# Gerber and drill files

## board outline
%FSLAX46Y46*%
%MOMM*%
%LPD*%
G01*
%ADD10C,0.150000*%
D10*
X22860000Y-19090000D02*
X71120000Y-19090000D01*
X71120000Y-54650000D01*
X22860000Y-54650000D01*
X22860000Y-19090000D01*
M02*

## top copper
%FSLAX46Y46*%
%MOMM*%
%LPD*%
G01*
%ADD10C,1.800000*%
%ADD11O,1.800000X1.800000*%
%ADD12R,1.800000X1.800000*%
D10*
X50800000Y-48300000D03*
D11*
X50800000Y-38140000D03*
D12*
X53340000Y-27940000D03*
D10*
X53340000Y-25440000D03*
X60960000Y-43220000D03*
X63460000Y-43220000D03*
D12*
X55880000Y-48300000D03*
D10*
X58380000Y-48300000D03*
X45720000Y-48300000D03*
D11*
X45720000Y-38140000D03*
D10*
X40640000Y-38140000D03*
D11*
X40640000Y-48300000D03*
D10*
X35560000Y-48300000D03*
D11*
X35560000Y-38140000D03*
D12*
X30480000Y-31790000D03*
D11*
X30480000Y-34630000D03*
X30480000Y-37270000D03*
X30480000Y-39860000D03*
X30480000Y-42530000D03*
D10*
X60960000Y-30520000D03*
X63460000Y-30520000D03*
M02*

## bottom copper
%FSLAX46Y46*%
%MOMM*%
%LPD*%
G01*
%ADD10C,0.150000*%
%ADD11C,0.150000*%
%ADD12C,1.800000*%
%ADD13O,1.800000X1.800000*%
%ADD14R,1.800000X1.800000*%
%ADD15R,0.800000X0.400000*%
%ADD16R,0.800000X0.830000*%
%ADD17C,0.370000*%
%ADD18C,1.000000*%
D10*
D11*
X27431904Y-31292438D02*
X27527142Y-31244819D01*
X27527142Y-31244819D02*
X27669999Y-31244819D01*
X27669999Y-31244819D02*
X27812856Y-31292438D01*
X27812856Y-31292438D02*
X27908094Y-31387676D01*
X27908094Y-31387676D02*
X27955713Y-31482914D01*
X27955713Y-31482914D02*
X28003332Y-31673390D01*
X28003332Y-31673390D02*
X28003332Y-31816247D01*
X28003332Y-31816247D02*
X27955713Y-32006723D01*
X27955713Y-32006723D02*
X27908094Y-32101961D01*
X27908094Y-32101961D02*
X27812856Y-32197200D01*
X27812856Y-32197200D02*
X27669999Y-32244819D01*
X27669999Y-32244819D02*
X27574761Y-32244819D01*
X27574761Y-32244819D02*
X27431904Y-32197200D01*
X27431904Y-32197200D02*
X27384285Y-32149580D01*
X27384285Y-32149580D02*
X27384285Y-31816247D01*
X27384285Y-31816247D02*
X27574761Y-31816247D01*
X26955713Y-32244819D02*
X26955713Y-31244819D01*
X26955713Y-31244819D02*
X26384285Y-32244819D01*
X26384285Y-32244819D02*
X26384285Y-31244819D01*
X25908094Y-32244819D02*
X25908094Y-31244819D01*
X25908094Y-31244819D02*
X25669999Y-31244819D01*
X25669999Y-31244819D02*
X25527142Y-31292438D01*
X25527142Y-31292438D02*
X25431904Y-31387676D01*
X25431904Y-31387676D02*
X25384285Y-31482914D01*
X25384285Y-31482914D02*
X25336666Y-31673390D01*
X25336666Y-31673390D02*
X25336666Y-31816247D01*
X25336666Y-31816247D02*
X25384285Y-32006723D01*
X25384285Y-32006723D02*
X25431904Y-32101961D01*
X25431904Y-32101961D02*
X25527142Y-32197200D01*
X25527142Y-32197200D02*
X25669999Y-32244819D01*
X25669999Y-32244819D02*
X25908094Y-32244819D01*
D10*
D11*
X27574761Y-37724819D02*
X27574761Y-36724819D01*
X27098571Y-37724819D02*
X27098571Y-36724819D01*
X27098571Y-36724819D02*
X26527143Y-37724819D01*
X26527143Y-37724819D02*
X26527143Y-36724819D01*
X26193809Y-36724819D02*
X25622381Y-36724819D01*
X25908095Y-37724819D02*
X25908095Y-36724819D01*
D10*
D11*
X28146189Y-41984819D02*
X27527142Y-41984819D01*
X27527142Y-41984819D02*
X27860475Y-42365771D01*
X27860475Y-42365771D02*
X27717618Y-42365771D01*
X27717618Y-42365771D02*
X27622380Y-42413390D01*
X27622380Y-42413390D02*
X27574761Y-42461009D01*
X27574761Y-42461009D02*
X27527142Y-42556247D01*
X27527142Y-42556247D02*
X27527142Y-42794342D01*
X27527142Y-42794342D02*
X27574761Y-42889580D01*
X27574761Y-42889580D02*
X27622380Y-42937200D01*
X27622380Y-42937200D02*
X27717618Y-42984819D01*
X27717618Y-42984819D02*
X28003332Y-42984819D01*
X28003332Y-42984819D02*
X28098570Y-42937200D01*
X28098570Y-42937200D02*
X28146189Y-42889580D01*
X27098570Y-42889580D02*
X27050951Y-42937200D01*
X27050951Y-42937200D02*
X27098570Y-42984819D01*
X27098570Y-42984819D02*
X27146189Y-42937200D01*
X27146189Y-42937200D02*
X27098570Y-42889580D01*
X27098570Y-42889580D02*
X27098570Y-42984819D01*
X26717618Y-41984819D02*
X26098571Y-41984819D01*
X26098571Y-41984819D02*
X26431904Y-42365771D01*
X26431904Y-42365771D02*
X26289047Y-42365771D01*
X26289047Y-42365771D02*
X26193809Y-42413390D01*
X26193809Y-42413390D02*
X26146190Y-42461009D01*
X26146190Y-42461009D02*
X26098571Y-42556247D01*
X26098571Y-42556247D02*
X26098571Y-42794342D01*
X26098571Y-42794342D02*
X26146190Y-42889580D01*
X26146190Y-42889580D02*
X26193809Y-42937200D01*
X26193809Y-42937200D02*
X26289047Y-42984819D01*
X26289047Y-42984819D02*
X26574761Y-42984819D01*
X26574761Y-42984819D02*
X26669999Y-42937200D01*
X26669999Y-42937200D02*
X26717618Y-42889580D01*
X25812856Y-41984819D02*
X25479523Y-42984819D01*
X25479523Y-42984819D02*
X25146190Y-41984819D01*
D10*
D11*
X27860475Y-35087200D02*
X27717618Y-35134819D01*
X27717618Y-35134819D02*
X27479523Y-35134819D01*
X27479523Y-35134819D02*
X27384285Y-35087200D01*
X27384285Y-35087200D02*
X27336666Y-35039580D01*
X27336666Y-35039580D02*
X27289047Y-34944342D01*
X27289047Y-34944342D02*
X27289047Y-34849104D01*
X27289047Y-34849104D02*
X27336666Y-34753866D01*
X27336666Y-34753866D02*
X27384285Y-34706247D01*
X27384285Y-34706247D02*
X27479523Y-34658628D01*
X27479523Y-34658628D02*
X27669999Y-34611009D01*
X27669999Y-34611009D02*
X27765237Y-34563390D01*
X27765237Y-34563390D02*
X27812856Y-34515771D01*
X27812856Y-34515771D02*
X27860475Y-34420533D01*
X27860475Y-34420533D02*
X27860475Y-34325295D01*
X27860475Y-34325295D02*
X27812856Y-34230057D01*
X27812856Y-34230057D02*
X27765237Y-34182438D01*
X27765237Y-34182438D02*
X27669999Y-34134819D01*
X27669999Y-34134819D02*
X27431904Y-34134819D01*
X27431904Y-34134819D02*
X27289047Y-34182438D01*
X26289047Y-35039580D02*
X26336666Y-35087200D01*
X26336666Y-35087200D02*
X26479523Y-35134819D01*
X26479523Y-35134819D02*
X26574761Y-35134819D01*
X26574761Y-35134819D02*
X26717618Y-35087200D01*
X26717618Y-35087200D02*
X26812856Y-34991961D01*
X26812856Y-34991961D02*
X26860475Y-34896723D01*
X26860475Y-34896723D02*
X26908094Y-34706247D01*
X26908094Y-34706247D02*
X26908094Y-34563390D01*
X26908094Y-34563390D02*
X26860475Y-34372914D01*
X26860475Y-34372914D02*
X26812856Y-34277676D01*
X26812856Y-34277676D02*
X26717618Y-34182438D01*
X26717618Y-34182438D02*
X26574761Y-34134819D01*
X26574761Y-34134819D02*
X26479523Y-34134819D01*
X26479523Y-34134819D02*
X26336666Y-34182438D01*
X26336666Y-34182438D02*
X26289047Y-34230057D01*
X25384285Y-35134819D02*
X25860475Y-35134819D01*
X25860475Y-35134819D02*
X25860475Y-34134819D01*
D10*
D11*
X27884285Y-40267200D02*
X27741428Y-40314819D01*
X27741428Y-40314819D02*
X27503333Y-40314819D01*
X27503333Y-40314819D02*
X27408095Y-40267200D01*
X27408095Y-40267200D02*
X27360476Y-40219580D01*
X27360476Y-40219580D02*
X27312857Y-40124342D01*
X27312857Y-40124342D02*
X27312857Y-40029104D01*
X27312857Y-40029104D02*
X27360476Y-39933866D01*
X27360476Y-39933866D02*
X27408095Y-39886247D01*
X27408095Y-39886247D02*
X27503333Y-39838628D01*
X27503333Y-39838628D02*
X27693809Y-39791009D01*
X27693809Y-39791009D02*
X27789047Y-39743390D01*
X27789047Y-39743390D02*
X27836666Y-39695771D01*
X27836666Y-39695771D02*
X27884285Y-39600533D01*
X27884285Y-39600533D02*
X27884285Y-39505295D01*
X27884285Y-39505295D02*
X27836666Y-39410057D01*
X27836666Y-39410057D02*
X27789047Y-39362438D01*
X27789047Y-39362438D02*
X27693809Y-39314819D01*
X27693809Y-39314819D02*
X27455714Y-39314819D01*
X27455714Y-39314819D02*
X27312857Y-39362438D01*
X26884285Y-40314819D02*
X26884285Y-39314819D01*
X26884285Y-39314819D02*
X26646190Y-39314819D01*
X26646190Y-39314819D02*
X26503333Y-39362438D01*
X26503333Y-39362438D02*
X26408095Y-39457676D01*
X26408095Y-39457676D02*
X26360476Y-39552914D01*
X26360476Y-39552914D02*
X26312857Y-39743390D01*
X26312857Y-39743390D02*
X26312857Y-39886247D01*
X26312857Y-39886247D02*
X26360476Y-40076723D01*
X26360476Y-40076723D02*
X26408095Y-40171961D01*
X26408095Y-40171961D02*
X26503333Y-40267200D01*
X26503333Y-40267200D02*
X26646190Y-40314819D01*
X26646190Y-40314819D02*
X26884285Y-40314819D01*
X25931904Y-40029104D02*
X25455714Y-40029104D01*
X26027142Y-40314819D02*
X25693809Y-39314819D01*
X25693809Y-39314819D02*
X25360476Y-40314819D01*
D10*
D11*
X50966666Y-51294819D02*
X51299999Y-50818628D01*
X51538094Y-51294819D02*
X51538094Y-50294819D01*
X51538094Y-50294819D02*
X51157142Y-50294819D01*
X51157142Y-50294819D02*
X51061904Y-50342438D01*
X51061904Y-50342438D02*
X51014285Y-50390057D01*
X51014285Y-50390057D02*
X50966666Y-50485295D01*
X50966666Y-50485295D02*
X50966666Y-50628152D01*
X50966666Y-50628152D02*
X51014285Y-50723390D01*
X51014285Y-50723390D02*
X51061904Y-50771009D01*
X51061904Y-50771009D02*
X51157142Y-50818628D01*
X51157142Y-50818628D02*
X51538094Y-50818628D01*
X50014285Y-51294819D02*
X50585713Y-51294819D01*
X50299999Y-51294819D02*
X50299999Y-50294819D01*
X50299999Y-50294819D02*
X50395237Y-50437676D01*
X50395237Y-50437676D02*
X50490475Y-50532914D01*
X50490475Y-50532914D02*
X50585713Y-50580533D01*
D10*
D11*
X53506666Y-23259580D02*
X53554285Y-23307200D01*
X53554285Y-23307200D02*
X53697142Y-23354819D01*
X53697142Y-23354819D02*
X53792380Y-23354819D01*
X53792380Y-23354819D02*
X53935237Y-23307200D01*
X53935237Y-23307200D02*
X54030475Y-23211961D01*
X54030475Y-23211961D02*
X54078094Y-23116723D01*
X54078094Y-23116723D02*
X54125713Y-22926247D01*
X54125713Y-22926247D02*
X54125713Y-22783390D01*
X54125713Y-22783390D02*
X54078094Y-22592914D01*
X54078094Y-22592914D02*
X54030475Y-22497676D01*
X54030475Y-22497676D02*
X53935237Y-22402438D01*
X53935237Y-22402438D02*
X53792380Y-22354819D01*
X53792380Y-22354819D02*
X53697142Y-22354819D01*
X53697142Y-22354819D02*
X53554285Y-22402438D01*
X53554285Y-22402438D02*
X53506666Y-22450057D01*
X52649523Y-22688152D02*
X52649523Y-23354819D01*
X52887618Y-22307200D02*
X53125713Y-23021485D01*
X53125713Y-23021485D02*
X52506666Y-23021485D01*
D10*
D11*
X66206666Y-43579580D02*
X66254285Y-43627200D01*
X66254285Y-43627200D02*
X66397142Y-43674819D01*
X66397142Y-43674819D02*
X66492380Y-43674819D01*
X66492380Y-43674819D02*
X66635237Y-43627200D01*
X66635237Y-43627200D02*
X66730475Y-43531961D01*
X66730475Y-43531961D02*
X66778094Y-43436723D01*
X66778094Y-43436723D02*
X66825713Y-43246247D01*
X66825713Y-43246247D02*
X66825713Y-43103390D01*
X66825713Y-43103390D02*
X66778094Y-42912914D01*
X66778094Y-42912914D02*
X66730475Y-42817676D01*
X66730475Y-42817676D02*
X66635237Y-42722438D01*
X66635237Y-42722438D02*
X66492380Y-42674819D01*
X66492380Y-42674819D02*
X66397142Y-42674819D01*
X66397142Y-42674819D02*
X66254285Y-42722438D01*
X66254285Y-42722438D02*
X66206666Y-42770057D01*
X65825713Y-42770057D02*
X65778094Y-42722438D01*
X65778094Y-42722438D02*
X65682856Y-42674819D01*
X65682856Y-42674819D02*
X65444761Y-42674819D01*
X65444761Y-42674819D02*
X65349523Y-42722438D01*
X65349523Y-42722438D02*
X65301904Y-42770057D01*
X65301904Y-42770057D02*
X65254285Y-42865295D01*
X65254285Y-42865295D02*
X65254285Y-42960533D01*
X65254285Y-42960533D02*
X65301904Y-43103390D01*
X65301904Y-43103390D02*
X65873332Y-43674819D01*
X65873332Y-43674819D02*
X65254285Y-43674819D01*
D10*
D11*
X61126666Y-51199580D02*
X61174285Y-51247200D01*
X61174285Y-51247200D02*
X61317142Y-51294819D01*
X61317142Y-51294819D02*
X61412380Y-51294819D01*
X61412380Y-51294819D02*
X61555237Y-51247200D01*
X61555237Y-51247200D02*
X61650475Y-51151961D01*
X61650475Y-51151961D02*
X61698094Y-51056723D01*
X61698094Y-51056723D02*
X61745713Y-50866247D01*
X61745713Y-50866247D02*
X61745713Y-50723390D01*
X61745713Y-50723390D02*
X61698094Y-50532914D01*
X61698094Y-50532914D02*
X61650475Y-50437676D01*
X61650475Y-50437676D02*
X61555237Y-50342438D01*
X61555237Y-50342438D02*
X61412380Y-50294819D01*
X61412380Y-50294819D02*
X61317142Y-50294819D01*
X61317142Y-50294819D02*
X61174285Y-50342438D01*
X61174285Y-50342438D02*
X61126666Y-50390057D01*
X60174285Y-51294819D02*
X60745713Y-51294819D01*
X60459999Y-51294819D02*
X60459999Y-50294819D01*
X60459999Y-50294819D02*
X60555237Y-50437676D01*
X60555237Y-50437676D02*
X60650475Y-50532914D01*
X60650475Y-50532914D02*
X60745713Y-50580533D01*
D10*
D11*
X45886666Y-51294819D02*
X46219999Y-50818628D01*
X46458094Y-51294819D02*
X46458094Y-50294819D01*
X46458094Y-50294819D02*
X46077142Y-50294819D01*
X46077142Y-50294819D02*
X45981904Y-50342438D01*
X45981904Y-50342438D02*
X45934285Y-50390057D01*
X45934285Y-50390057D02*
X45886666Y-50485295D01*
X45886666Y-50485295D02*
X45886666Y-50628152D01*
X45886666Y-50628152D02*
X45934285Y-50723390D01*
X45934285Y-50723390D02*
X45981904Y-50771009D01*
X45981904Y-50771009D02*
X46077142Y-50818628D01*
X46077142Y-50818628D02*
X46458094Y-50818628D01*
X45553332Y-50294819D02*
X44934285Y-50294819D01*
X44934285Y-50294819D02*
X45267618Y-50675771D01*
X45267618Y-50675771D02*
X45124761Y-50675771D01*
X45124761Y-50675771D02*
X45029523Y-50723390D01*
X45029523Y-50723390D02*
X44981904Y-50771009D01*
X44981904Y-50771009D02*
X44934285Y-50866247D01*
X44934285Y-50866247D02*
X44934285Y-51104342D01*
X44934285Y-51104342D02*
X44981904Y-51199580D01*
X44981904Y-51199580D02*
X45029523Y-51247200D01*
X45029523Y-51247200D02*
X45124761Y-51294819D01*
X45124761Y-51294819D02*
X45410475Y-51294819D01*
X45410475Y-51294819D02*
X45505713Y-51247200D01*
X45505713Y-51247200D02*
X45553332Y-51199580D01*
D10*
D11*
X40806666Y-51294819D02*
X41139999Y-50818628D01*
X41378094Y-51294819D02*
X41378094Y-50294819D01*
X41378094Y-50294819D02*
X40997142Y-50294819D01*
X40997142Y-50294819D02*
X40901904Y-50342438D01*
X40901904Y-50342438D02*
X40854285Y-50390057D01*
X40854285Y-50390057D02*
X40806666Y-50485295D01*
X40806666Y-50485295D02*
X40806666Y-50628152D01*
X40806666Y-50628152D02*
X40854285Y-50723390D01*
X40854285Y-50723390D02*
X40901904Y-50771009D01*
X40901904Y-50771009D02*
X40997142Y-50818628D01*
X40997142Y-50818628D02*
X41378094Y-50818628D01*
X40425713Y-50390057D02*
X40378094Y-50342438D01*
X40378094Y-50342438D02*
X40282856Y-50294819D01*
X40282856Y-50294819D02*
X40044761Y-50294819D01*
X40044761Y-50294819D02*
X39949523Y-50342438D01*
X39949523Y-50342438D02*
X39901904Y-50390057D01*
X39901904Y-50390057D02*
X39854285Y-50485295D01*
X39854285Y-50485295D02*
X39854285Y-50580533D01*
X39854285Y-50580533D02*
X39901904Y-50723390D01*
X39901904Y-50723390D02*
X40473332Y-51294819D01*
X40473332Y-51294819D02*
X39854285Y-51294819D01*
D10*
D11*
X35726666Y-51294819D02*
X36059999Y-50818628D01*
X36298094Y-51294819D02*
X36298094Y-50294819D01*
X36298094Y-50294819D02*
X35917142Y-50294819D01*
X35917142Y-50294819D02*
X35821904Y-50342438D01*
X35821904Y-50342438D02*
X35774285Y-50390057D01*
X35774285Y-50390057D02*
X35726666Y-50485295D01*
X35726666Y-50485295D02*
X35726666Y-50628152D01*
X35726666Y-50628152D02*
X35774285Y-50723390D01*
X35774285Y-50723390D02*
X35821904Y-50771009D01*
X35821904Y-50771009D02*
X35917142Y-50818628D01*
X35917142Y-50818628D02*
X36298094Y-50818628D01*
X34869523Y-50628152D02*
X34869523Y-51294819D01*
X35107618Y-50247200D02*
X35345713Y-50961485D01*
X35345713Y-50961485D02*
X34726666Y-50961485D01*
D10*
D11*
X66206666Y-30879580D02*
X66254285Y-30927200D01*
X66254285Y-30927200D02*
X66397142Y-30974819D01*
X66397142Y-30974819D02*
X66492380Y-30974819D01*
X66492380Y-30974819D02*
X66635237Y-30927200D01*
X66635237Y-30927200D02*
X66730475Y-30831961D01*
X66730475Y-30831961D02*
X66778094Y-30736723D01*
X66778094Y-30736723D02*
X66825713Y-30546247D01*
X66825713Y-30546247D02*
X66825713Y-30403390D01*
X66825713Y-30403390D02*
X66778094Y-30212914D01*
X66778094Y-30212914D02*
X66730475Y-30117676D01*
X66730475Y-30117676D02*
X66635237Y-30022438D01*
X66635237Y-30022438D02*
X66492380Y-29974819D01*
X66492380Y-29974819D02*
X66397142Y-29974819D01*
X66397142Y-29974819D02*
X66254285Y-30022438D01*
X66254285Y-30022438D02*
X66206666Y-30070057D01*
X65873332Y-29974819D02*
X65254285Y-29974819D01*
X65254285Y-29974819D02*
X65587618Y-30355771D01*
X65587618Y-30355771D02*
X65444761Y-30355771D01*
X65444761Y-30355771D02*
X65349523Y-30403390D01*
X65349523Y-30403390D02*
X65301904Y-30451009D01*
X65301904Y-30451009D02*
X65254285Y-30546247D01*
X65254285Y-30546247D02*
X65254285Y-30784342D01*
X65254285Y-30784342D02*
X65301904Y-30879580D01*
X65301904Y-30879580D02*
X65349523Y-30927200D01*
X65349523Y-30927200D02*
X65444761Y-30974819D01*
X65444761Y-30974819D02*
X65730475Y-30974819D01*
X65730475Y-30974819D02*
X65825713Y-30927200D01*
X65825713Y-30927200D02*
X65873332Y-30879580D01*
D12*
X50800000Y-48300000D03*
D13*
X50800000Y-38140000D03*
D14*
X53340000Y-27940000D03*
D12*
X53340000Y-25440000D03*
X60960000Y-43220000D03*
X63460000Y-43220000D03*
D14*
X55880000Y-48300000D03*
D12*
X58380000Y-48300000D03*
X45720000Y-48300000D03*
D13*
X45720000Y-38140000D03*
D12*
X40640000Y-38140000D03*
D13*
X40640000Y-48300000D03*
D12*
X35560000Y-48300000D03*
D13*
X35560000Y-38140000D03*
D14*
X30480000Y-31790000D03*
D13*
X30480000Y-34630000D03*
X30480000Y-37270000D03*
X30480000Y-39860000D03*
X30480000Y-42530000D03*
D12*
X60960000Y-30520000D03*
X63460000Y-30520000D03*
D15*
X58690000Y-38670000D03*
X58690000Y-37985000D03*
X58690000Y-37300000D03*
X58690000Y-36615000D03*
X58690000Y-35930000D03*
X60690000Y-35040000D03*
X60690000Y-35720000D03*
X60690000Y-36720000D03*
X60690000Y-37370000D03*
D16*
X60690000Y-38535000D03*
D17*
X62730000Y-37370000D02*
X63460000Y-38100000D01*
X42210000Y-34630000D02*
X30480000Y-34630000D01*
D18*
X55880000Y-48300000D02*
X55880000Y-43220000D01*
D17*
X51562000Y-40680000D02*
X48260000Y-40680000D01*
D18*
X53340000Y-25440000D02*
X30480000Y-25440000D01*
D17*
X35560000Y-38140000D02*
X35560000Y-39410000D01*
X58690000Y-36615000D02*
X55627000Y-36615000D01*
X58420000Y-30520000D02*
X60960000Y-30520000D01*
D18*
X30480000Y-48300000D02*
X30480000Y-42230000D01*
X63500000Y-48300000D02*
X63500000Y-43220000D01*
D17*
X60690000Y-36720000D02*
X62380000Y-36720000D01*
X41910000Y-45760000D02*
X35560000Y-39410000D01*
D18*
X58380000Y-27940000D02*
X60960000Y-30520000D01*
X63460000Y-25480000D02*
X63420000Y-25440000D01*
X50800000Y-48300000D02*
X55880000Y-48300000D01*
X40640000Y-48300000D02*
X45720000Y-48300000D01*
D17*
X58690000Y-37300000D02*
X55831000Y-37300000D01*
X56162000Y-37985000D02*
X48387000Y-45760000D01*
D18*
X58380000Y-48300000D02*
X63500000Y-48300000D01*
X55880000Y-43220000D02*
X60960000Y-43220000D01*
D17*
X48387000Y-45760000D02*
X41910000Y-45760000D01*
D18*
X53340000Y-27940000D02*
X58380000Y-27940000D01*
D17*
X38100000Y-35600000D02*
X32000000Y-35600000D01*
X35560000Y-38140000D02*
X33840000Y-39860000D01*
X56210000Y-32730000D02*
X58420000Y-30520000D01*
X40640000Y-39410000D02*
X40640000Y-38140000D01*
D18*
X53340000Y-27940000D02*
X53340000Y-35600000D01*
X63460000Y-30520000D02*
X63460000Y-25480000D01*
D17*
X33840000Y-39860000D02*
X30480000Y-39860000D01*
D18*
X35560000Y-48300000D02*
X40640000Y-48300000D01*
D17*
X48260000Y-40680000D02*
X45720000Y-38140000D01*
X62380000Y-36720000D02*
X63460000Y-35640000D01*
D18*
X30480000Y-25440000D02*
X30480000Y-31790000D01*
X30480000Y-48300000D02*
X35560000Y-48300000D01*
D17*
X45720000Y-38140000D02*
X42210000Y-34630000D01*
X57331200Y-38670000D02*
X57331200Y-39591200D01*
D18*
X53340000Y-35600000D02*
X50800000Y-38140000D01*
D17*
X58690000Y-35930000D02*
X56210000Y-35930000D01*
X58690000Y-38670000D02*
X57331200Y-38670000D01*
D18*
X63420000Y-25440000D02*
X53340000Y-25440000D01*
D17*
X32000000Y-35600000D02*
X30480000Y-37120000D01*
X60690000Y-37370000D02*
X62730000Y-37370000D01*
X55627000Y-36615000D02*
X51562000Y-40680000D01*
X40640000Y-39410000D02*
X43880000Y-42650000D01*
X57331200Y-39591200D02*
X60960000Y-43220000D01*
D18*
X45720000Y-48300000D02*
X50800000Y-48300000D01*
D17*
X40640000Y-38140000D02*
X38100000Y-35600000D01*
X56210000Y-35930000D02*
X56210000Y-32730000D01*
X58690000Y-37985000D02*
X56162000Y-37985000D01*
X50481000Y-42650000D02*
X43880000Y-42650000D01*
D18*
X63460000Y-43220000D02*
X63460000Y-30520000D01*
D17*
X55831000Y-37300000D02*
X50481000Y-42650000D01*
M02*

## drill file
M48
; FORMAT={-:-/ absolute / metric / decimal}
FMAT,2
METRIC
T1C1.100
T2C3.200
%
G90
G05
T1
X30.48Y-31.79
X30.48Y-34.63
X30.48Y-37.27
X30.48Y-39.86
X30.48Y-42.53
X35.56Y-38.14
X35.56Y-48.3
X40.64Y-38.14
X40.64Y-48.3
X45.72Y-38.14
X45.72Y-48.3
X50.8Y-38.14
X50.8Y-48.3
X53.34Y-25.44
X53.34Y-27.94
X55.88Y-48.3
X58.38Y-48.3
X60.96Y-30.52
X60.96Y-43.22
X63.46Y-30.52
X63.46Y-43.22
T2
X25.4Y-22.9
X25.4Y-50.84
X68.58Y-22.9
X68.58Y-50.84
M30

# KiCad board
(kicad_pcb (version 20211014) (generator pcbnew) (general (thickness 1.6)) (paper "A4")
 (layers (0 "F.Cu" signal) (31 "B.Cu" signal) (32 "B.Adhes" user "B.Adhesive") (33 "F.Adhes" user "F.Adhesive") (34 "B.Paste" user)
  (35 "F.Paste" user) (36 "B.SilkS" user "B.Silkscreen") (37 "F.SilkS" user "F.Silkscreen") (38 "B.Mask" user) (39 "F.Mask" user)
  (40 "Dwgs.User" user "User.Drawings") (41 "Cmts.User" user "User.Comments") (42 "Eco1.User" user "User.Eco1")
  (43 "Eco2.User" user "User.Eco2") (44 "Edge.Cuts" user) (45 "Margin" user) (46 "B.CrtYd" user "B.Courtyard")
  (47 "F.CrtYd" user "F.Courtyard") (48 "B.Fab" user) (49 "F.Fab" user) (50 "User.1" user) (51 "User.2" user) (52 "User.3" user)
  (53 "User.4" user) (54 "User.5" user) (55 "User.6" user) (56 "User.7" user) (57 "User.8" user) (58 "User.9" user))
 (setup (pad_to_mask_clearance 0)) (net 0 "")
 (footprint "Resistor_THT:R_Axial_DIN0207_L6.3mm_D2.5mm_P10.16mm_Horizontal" (layer "F.Cu") (at 50.8 48.3 90)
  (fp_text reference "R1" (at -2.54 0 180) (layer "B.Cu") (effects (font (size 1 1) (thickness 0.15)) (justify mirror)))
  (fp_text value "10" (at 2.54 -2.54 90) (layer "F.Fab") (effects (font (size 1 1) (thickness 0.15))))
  (pad "1" thru_hole circle (at 0 0 90) (size 1.8 1.8) (drill 1.1) (layers *.Cu *.Mask))
  (pad "2" thru_hole oval (at 10.16 0 90) (size 1.8 1.8) (drill 1.1) (layers *.Cu *.Mask)))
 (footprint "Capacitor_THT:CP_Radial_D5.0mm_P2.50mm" (layer "F.Cu") (at 53.34 27.94 90)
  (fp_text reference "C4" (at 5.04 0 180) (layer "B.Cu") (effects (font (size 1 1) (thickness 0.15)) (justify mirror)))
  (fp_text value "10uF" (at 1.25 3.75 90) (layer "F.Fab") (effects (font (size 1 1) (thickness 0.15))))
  (pad "1" thru_hole rect (at 0 0 90) (size 1.8 1.8) (drill 1.1) (layers *.Cu *.Mask))
  (pad "2" thru_hole circle (at 2.5 0 90) (size 1.8 1.8) (drill 1.1) (layers *.Cu *.Mask)))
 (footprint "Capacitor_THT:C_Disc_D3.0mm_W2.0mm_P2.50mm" (layer "F.Cu") (at 60.96 43.22)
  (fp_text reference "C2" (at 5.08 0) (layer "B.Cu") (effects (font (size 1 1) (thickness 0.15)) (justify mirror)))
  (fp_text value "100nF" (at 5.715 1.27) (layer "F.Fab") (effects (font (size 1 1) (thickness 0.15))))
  (pad "1" thru_hole circle (at 0 0) (size 1.8 1.8) (drill 1.1) (layers *.Cu *.Mask))
  (pad "2" thru_hole circle (at 2.5 0) (size 1.8 1.8) (drill 1.1) (layers *.Cu *.Mask)))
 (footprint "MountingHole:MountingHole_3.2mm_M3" (layer "F.Cu") (at 25.4 22.9)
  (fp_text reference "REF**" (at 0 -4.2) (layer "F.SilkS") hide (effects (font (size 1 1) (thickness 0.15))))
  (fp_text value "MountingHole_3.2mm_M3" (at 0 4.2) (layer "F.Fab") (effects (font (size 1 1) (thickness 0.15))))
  (pad "" np_thru_hole circle (at 0 0) (size 3.2 3.2) (drill 3.2) (layers *.Cu *.Mask)))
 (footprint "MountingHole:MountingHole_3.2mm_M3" (layer "F.Cu") (at 25.4 50.84)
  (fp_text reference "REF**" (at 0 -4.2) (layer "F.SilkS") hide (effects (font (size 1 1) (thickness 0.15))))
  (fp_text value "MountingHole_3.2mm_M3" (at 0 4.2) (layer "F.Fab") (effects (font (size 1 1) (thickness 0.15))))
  (pad "" np_thru_hole circle (at 0 0) (size 3.2 3.2) (drill 3.2) (layers *.Cu *.Mask)))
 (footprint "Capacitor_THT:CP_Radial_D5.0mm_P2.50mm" (layer "F.Cu") (at 55.88 48.3)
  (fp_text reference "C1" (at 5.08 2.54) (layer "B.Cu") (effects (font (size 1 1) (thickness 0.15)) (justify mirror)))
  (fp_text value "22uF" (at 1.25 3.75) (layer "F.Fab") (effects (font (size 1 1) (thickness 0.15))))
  (pad "1" thru_hole rect (at 0 0) (size 1.8 1.8) (drill 1.1) (layers *.Cu *.Mask))
  (pad "2" thru_hole circle (at 2.5 0) (size 1.8 1.8) (drill 1.1) (layers *.Cu *.Mask)))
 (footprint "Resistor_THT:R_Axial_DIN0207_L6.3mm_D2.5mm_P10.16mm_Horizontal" (layer "F.Cu") (at 45.72 48.3 90)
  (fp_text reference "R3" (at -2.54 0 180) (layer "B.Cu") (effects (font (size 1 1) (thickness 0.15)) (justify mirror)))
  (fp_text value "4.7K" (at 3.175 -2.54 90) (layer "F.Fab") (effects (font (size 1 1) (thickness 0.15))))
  (pad "1" thru_hole circle (at 0 0 90) (size 1.8 1.8) (drill 1.1) (layers *.Cu *.Mask))
  (pad "2" thru_hole oval (at 10.16 0 90) (size 1.8 1.8) (drill 1.1) (layers *.Cu *.Mask)))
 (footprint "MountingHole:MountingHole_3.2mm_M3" (layer "F.Cu") (at 68.58 22.9)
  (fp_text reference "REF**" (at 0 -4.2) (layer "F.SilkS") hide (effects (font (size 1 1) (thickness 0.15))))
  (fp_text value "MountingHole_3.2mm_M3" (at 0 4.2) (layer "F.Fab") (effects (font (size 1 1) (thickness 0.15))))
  (pad "" np_thru_hole circle (at 0 0) (size 3.2 3.2) (drill 3.2) (layers *.Cu *.Mask)))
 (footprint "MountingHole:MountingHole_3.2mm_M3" (layer "F.Cu") (at 68.58 50.84)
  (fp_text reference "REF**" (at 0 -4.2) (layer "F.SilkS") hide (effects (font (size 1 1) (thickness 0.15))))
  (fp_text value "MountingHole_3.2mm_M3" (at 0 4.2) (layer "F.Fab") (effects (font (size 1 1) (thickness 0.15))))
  (pad "" np_thru_hole circle (at 0 0) (size 3.2 3.2) (drill 3.2) (layers *.Cu *.Mask)))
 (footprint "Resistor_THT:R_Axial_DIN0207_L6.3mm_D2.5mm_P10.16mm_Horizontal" (layer "F.Cu") (at 40.64 38.14 -90)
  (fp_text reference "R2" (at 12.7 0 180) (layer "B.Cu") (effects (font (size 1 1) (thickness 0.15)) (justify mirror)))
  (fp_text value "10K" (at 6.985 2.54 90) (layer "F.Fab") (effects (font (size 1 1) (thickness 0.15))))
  (pad "1" thru_hole circle (at 0 0 270) (size 1.8 1.8) (drill 1.1) (layers *.Cu *.Mask))
  (pad "2" thru_hole oval (at 10.16 0 270) (size 1.8 1.8) (drill 1.1) (layers *.Cu *.Mask)))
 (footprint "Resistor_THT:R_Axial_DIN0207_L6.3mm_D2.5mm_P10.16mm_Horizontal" (layer "F.Cu") (at 35.56 48.3 90)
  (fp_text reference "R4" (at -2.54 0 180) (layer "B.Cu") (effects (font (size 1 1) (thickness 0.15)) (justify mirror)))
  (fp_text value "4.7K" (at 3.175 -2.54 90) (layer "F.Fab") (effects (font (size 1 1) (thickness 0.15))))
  (pad "1" thru_hole circle (at 0 0 90) (size 1.8 1.8) (drill 1.1) (layers *.Cu *.Mask))
  (pad "2" thru_hole oval (at 10.16 0 90) (size 1.8 1.8) (drill 1.1) (layers *.Cu *.Mask)))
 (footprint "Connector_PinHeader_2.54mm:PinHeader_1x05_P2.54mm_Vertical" (layer "F.Cu") (at 30.48 31.79)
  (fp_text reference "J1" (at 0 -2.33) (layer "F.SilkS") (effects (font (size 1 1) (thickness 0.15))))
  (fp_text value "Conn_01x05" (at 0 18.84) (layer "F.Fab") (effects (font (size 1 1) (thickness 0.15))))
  (pad "1" thru_hole rect (at 0 0) (size 1.8 1.8) (drill 1.1) (layers *.Cu *.Mask))
  (pad "2" thru_hole oval (at 0 2.84) (size 1.8 1.8) (drill 1.1) (layers *.Cu *.Mask))
  (pad "3" thru_hole oval (at 0 5.48) (size 1.8 1.8) (drill 1.1) (layers *.Cu *.Mask))
  (pad "4" thru_hole oval (at 0 8.07) (size 1.8 1.8) (drill 1.1) (layers *.Cu *.Mask))
  (pad "5" thru_hole oval (at 0 10.74) (size 1.8 1.8) (drill 1.1) (layers *.Cu *.Mask)))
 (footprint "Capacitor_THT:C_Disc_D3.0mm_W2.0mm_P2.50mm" (layer "F.Cu") (at 60.96 30.52)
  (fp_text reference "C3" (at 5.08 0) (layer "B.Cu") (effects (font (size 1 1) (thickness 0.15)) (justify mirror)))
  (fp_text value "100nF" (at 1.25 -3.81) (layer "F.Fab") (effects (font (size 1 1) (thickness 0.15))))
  (pad "1" thru_hole circle (at 0 0) (size 1.8 1.8) (drill 1.1) (layers *.Cu *.Mask))
  (pad "2" thru_hole circle (at 2.5 0) (size 1.8 1.8) (drill 1.1) (layers *.Cu *.Mask)))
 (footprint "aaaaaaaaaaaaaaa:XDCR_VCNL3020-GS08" (layer "B.Cu") (at 59.69 36.87)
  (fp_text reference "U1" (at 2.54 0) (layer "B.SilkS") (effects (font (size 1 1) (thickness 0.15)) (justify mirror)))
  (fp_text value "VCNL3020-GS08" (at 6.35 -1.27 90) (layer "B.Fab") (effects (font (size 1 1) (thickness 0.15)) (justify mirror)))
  (pad "1" smd rect (at -1 1.8 270) (size 0.4 0.8) (layers "B.Cu" "B.Paste" "B.Mask"))
  (pad "2" smd rect (at -1 1.115 90) (size 0.4 0.8) (layers "B.Cu" "B.Paste" "B.Mask"))
  (pad "3" smd rect (at -1 0.43 90) (size 0.4 0.8) (layers "B.Cu" "B.Paste" "B.Mask"))
  (pad "4" smd rect (at -1 -0.255 90) (size 0.4 0.8) (layers "B.Cu" "B.Paste" "B.Mask"))
  (pad "5" smd rect (at -1 -0.94 90) (size 0.4 0.8) (layers "B.Cu" "B.Paste" "B.Mask"))
  (pad "6" smd rect (at 1 -1.83 270) (size 0.4 0.8) (layers "B.Cu" "B.Paste" "B.Mask"))
  (pad "7" smd rect (at 1 -1.15 270) (size 0.4 0.8) (layers "B.Cu" "B.Paste" "B.Mask"))
  (pad "8" smd rect (at 1 -0.15 270) (size 0.4 0.8) (layers "B.Cu" "B.Paste" "B.Mask"))
  (pad "9" smd rect (at 1 0.5 270) (size 0.4 0.8) (layers "B.Cu" "B.Paste" "B.Mask"))
  (pad "10" smd rect (at 1 1.665 270) (size 0.83 0.8) (layers "B.Cu" "B.Paste" "B.Mask")))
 (gr_rect (start 22.86 19.09) (end 71.12 54.65) (layer "Edge.Cuts") (width 0.15) (fill none))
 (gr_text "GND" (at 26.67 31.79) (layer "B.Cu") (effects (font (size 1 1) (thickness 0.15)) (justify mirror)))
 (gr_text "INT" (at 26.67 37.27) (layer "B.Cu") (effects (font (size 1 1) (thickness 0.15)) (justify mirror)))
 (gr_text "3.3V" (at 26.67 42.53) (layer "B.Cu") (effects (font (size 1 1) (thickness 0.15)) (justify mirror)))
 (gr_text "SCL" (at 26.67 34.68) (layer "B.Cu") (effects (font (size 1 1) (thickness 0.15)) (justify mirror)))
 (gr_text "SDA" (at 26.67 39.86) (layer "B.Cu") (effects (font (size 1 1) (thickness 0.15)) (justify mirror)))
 (segment (start 62.73 37.37) (end 63.46 38.1) (width 0.37) (layer "B.Cu") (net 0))
 (segment (start 42.21 34.63) (end 30.48 34.63) (width 0.37) (layer "B.Cu") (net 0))
 (segment (start 55.88 48.3) (end 55.88 43.22) (width 1) (layer "B.Cu") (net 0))
 (segment (start 51.562 40.68) (end 48.26 40.68) (width 0.37) (layer "B.Cu") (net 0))
 (segment (start 53.34 25.44) (end 30.48 25.44) (width 1) (layer "B.Cu") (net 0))
 (segment (start 35.56 38.14) (end 35.56 39.41) (width 0.37) (layer "B.Cu") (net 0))
 (segment (start 58.69 36.615) (end 55.627 36.615) (width 0.37) (layer "B.Cu") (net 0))
 (segment (start 58.42 30.52) (end 60.96 30.52) (width 0.37) (layer "B.Cu") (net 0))
 (segment (start 30.48 48.3) (end 30.48 42.23) (width 1) (layer "B.Cu") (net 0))
 (segment (start 63.5 48.3) (end 63.5 43.22) (width 1) (layer "B.Cu") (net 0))
 (segment (start 60.69 36.72) (end 62.38 36.72) (width 0.37) (layer "B.Cu") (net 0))
 (segment (start 41.91 45.76) (end 35.56 39.41) (width 0.37) (layer "B.Cu") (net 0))
 (segment (start 58.38 27.94) (end 60.96 30.52) (width 1) (layer "B.Cu") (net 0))
 (segment (start 63.46 25.48) (end 63.42 25.44) (width 1) (layer "B.Cu") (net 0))
 (segment (start 50.8 48.3) (end 55.88 48.3) (width 1) (layer "B.Cu") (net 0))
 (segment (start 40.64 48.3) (end 45.72 48.3) (width 1) (layer "B.Cu") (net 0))
 (segment (start 58.69 37.3) (end 55.831 37.3) (width 0.37) (layer "B.Cu") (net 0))
 (segment (start 56.162 37.985) (end 48.387 45.76) (width 0.37) (layer "B.Cu") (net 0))
 (segment (start 58.38 48.3) (end 63.5 48.3) (width 1) (layer "B.Cu") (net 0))
 (segment (start 55.88 43.22) (end 60.96 43.22) (width 1) (layer "B.Cu") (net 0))
 (segment (start 48.387 45.76) (end 41.91 45.76) (width 0.37) (layer "B.Cu") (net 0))
 (segment (start 53.34 27.94) (end 58.38 27.94) (width 1) (layer "B.Cu") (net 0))
 (segment (start 38.1 35.6) (end 32 35.6) (width 0.37) (layer "B.Cu") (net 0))
 (segment (start 35.56 38.14) (end 33.84 39.86) (width 0.37) (layer "B.Cu") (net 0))
 (segment (start 56.21 32.73) (end 58.42 30.52) (width 0.37) (layer "B.Cu") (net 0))
 (segment (start 40.64 39.41) (end 40.64 38.14) (width 0.37) (layer "B.Cu") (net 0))
 (segment (start 53.34 27.94) (end 53.34 35.6) (width 1) (layer "B.Cu") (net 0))
 (segment (start 63.46 30.52) (end 63.46 25.48) (width 1) (layer "B.Cu") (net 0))
 (segment (start 33.84 39.86) (end 30.48 39.86) (width 0.37) (layer "B.Cu") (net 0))
 (segment (start 35.56 48.3) (end 40.64 48.3) (width 1) (layer "B.Cu") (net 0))
 (segment (start 48.26 40.68) (end 45.72 38.14) (width 0.37) (layer "B.Cu") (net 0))
 (segment (start 62.38 36.72) (end 63.46 35.64) (width 0.37) (layer "B.Cu") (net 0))
 (segment (start 30.48 25.44) (end 30.48 31.79) (width 1) (layer "B.Cu") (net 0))
 (segment (start 30.48 48.3) (end 35.56 48.3) (width 1) (layer "B.Cu") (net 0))
 (segment (start 45.72 38.14) (end 42.21 34.63) (width 0.37) (layer "B.Cu") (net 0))
 (segment (start 57.3312 38.67) (end 57.3312 39.5912) (width 0.37) (layer "B.Cu") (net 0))
 (segment (start 53.34 35.6) (end 50.8 38.14) (width 1) (layer "B.Cu") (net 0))
 (segment (start 58.69 35.93) (end 56.21 35.93) (width 0.37) (layer "B.Cu") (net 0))
 (segment (start 58.69 38.67) (end 57.3312 38.67) (width 0.37) (layer "B.Cu") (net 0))
 (segment (start 63.42 25.44) (end 53.34 25.44) (width 1) (layer "B.Cu") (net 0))
 (segment (start 32 35.6) (end 30.48 37.12) (width 0.37) (layer "B.Cu") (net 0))
 (segment (start 60.69 37.37) (end 62.73 37.37) (width 0.37) (layer "B.Cu") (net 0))
 (segment (start 55.627 36.615) (end 51.562 40.68) (width 0.37) (layer "B.Cu") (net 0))
 (segment (start 40.64 39.41) (end 43.88 42.65) (width 0.37) (layer "B.Cu") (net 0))
 (segment (start 57.3312 39.5912) (end 60.96 43.22) (width 0.37) (layer "B.Cu") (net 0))
 (segment (start 45.72 48.3) (end 50.8 48.3) (width 1) (layer "B.Cu") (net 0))
 (segment (start 40.64 38.14) (end 38.1 35.6) (width 0.37) (layer "B.Cu") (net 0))
 (segment (start 56.21 35.93) (end 56.21 32.73) (width 0.37) (layer "B.Cu") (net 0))
 (segment (start 58.69 37.985) (end 56.162 37.985) (width 0.37) (layer "B.Cu") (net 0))
 (segment (start 50.481 42.65) (end 43.88 42.65) (width 0.37) (layer "B.Cu") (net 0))
 (segment (start 63.46 43.22) (end 63.46 30.52) (width 1) (layer "B.Cu") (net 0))
 (segment (start 55.831 37.3) (end 50.481 42.65) (width 0.37) (layer "B.Cu") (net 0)))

